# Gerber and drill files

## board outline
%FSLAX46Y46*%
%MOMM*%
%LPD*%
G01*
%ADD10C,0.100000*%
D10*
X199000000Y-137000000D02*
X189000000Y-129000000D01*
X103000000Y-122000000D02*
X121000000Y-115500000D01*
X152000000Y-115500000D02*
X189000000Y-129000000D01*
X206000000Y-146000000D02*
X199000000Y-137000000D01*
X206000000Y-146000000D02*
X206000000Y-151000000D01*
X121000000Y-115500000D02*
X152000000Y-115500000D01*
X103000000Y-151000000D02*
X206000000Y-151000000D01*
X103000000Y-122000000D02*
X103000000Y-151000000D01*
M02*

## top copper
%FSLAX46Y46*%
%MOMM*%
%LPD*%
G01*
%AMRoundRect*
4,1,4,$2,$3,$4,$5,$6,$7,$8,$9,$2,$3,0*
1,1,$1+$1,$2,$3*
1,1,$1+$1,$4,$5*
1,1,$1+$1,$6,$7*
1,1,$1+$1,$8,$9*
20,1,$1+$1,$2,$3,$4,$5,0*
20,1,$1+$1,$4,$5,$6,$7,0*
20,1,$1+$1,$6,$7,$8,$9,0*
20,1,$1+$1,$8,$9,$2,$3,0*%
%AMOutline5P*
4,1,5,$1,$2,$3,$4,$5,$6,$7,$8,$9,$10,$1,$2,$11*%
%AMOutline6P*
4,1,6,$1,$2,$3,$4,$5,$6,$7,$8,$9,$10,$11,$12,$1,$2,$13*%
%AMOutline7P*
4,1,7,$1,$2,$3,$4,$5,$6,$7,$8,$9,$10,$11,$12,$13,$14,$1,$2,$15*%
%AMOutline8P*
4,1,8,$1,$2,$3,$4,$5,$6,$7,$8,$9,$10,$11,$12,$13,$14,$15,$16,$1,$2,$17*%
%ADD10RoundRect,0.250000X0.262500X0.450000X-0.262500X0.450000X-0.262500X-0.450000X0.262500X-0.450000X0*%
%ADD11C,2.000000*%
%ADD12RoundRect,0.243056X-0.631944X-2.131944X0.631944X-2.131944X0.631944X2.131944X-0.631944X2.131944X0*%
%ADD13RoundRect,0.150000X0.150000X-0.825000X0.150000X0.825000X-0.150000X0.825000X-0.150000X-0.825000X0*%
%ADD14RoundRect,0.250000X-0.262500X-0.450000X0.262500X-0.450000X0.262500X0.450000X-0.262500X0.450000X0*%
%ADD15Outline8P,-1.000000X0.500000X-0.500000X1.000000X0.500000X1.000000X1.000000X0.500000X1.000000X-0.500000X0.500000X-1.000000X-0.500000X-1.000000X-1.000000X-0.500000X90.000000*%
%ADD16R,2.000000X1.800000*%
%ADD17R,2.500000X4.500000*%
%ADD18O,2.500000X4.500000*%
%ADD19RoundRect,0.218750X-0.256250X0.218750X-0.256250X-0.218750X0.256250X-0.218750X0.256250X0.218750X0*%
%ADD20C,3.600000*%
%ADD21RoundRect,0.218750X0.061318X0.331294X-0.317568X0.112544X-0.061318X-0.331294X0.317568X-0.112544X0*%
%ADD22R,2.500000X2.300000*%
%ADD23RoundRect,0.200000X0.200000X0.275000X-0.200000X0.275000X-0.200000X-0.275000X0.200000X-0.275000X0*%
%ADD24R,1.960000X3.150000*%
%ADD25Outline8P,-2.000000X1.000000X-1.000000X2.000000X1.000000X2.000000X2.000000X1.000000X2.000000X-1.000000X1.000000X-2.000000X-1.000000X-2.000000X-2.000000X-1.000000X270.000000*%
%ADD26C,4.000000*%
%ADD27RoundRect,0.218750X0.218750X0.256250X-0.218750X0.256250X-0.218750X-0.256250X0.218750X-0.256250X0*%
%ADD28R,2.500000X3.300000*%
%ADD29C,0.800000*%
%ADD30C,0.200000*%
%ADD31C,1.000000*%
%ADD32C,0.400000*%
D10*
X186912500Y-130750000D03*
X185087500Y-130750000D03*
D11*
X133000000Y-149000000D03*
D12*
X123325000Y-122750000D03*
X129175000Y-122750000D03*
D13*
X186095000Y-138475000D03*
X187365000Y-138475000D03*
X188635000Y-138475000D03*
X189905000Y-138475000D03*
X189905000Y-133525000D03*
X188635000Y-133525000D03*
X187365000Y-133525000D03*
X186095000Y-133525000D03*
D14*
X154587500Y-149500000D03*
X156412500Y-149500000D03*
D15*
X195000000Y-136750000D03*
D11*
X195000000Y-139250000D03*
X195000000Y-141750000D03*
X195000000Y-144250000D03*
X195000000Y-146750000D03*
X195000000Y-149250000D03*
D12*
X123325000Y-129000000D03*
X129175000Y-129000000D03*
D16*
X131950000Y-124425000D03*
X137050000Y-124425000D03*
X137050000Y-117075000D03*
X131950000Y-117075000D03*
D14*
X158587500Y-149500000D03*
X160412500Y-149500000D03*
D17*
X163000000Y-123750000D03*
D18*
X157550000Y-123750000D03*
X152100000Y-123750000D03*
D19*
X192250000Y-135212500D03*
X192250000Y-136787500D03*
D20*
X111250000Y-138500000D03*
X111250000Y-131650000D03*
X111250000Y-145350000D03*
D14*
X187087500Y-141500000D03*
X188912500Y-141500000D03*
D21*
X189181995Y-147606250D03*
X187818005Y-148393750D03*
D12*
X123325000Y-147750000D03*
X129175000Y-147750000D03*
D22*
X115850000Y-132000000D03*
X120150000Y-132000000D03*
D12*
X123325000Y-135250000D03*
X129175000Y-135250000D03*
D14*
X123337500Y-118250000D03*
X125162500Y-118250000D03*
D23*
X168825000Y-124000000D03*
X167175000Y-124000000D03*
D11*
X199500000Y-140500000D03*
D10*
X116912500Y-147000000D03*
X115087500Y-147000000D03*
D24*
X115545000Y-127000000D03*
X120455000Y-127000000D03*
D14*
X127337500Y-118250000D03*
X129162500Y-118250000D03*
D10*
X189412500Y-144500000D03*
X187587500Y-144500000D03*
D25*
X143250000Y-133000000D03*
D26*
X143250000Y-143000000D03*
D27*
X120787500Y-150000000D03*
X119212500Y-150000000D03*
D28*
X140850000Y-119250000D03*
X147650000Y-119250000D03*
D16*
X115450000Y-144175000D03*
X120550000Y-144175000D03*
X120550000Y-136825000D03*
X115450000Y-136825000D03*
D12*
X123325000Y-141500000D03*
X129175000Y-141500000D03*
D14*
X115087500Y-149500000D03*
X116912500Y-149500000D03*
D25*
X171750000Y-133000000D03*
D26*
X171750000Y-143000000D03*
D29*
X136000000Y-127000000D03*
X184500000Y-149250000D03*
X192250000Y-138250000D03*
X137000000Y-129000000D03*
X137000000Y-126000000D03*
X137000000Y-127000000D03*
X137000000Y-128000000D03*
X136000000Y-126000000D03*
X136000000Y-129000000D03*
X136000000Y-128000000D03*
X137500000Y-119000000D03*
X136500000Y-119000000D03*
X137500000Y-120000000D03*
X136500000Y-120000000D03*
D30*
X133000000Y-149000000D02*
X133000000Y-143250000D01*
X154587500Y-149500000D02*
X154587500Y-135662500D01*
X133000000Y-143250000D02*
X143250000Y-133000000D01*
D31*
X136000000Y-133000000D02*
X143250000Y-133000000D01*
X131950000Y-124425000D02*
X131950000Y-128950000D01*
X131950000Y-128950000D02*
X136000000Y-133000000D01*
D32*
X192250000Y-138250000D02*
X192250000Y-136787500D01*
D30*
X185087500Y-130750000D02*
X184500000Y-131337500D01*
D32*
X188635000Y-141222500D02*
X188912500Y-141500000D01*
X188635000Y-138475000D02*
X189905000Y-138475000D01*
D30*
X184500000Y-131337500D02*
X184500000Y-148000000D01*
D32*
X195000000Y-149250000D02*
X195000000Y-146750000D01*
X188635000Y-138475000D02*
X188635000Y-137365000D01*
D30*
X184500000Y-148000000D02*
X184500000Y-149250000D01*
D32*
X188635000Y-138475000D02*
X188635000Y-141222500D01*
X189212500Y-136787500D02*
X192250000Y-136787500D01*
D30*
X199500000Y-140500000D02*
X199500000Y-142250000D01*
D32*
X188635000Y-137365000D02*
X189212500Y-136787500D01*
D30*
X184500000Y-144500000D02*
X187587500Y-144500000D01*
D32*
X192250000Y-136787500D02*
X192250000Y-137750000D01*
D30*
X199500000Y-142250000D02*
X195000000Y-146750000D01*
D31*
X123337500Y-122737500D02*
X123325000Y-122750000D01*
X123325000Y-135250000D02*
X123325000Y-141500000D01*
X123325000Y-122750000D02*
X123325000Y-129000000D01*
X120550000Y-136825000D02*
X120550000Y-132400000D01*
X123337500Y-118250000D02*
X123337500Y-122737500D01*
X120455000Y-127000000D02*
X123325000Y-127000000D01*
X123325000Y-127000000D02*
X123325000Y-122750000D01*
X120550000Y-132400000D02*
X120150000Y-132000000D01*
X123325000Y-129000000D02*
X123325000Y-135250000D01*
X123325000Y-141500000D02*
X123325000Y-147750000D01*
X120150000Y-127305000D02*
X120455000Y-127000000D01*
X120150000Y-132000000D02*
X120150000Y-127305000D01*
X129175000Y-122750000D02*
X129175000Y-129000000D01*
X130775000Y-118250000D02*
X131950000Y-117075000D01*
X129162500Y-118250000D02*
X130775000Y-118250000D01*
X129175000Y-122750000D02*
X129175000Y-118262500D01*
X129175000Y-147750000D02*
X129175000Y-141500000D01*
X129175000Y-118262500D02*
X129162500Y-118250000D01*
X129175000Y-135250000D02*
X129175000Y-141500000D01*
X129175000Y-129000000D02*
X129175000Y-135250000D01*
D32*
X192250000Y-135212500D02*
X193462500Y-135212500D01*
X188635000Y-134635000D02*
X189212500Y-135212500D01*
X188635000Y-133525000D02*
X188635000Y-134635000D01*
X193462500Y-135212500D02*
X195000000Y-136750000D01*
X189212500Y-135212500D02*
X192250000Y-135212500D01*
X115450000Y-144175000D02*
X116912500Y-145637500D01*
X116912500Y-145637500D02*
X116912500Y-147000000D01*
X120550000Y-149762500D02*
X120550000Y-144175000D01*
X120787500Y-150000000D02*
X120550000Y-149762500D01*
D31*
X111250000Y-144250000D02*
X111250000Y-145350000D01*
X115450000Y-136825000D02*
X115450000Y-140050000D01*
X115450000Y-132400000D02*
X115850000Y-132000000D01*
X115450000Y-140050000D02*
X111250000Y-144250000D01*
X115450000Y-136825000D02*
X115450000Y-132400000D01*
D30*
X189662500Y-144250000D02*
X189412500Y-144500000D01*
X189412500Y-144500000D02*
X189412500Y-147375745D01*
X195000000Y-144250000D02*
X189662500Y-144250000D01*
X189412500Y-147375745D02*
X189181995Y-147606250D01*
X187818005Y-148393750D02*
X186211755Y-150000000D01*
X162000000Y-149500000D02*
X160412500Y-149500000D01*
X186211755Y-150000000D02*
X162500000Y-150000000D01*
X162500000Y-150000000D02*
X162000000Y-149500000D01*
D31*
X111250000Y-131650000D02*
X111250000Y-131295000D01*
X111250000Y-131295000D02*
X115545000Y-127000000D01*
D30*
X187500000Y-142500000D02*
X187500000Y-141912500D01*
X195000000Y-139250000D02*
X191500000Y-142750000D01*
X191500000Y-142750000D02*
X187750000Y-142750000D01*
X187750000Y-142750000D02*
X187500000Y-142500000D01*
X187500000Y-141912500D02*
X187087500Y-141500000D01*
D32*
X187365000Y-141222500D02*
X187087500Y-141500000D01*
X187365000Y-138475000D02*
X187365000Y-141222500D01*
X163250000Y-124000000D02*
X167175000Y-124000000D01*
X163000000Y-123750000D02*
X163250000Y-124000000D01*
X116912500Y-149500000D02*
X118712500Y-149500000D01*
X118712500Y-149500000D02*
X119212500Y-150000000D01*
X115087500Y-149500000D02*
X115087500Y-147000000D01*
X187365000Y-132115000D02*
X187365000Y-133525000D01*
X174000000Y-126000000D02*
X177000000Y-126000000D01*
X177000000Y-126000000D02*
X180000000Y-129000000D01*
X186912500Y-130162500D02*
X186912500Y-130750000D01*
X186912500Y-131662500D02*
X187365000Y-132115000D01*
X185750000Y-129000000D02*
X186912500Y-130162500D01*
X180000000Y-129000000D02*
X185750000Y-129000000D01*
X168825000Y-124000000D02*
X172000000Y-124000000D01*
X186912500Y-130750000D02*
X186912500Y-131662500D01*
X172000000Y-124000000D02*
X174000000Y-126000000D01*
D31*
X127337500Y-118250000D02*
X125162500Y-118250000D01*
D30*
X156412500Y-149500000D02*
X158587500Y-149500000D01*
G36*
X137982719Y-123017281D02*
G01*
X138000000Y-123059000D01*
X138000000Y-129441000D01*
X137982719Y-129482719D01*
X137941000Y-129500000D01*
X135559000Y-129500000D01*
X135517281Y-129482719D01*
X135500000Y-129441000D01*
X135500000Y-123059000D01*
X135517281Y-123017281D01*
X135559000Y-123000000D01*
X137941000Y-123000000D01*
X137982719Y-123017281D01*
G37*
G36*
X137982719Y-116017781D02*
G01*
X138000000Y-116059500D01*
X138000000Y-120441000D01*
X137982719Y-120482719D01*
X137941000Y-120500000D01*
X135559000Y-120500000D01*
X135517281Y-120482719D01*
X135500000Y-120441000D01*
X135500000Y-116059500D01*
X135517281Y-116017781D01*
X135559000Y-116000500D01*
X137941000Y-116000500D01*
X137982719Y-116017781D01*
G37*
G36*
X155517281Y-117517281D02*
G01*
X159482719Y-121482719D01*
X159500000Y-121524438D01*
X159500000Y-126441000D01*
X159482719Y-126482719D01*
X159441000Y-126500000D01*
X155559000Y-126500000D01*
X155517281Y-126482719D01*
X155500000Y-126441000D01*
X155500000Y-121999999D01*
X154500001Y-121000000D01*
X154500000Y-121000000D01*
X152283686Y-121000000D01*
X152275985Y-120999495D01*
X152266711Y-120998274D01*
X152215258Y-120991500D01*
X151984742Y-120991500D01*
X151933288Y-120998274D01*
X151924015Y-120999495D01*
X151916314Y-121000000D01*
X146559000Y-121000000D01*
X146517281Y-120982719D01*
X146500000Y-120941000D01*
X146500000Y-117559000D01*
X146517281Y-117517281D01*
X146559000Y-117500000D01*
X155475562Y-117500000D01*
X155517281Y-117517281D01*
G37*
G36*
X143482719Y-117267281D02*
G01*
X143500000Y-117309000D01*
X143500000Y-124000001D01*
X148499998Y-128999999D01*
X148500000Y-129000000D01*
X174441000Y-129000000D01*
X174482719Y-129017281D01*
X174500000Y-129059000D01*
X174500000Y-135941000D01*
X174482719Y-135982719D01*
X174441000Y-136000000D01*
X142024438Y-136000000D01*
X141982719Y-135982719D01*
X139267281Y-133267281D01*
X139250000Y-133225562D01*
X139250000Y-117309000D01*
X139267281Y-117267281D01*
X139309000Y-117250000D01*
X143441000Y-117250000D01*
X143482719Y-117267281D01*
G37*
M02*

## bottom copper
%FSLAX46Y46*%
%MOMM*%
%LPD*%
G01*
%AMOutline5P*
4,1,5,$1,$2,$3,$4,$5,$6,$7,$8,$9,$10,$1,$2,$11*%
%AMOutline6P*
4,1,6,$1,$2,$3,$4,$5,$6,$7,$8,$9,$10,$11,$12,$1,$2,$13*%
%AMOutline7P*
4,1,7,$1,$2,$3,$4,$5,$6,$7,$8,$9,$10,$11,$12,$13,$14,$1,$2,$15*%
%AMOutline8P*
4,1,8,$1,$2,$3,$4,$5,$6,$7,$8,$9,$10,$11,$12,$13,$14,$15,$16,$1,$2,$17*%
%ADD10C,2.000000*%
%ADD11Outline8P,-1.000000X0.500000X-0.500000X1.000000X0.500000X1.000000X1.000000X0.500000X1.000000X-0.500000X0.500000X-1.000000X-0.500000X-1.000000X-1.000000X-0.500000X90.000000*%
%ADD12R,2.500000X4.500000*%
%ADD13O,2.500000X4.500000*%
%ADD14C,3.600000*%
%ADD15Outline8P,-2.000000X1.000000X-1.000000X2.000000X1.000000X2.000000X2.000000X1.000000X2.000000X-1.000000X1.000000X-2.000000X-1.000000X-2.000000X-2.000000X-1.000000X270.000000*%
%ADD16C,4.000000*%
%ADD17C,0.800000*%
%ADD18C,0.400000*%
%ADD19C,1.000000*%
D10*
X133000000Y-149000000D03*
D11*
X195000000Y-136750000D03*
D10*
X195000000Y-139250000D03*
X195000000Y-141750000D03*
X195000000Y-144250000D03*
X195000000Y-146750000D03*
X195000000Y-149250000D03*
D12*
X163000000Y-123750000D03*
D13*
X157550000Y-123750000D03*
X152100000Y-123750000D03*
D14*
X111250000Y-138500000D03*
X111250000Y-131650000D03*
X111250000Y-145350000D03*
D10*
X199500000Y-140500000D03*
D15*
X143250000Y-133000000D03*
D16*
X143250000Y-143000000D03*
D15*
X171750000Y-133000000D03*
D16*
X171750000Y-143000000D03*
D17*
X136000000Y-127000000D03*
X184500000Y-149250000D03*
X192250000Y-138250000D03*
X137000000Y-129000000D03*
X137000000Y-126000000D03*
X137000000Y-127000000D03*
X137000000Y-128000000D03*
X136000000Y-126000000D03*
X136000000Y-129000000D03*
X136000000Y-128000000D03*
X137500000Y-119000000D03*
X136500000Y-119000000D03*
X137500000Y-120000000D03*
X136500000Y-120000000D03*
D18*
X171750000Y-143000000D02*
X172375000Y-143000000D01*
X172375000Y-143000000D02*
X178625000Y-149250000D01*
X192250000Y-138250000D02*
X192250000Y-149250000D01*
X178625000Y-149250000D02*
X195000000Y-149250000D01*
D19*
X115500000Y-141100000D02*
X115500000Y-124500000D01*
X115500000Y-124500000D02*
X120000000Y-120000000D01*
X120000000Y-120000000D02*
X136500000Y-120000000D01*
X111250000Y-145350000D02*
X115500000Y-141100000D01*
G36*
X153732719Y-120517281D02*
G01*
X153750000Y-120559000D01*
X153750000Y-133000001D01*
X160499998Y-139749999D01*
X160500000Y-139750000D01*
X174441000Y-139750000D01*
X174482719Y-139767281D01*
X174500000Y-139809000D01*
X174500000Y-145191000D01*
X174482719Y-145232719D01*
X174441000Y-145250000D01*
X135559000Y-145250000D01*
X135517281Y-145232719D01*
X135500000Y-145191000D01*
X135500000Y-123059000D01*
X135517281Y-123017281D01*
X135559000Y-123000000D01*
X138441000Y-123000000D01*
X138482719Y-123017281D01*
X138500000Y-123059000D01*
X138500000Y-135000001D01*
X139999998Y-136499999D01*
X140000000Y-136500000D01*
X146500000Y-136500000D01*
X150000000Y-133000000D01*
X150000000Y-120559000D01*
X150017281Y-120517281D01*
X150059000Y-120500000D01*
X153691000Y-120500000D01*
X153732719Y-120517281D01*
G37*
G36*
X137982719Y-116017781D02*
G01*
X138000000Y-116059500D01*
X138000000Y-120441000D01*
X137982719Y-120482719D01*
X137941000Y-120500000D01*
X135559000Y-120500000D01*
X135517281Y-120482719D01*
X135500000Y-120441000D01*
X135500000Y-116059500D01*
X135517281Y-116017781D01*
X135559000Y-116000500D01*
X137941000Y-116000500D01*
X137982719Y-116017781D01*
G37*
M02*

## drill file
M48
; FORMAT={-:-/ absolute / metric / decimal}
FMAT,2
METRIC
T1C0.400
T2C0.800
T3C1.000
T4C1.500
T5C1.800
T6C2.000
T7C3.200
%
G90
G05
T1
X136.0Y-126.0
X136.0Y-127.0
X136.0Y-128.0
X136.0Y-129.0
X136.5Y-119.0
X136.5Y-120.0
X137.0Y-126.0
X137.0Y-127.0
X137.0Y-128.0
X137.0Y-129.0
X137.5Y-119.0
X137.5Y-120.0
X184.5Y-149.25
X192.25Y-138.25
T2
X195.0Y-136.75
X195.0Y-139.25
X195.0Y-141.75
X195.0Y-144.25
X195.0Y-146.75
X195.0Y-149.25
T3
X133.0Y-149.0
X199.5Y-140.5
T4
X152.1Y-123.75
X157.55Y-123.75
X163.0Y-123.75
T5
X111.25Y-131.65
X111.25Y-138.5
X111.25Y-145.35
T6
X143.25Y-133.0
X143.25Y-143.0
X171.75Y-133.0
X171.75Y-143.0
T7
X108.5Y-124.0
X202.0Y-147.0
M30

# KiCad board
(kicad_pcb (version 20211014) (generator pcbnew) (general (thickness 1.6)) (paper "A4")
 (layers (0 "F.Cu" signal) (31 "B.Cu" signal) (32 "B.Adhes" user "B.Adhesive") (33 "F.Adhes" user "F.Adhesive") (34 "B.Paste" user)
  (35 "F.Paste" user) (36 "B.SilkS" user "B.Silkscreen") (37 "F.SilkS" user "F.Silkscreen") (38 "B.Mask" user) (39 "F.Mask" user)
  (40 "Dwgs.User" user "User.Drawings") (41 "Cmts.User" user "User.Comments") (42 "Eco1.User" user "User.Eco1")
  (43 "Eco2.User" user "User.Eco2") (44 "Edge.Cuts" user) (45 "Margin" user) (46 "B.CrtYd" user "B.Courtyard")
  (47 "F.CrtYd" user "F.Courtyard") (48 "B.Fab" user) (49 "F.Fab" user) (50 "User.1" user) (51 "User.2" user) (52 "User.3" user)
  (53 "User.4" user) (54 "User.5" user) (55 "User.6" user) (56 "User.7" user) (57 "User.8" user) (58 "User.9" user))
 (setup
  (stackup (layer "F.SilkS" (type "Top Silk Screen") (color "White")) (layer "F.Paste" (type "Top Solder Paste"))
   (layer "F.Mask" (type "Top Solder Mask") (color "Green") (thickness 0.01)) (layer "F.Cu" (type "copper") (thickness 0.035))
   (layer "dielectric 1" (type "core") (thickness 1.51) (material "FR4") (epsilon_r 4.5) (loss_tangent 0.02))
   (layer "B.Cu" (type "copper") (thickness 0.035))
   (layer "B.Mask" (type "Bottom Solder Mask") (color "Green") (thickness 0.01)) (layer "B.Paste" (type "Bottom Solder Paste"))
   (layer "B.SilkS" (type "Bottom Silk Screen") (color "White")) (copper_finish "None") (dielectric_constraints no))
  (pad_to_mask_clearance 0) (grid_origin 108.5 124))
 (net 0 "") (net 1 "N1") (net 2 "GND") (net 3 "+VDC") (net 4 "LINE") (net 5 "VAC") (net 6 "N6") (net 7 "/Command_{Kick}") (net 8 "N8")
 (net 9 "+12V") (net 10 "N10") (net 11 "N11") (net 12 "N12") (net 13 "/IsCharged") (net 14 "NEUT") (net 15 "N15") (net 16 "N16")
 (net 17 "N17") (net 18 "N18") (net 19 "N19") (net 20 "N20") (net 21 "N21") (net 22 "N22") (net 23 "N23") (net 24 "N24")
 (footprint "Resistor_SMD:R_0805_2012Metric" (layer "F.Cu") (at 186 130.75 180)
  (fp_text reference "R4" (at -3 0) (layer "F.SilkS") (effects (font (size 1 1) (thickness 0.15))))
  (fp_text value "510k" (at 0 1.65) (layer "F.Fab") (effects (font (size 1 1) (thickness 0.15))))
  (pad "1" smd roundrect (at -0.9125 0 180) (size 1.025 1.4) (layers "F.Cu" "F.Paste" "F.Mask") (roundrect_rratio 0.243902439) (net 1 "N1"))
  (pad "2" smd roundrect (at 0.9125 0 180) (size 1.025 1.4) (layers "F.Cu" "F.Paste" "F.Mask") (roundrect_rratio 0.243902439) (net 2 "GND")))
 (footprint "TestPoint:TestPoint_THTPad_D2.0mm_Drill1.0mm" (layer "F.Cu") (at 133 149)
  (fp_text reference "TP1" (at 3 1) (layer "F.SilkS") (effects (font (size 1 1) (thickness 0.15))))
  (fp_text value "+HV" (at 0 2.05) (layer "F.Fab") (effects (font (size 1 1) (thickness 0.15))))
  (pad "1" thru_hole circle (at 0 0) (size 2 2) (drill 1) (layers *.Cu *.Mask) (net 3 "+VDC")))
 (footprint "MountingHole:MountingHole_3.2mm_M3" (layer "F.Cu") (at 202 147)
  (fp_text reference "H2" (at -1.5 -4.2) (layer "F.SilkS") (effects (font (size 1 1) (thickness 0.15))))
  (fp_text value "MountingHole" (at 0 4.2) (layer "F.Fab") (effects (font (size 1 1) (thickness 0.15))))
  (pad "" np_thru_hole circle (at 0 0) (size 3.2 3.2) (drill 3.2) (layers *.Cu *.Mask)))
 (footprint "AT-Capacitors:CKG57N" (layer "F.Cu") (at 126.25 122.75)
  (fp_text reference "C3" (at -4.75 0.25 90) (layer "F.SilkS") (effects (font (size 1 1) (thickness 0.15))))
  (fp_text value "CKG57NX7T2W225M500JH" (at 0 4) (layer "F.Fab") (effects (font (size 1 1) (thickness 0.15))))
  (pad "1" smd roundrect (at -2.925 0) (size 1.75 4.75) (layers "F.Cu" "F.Paste" "F.Mask") (roundrect_rratio 0.1388891429) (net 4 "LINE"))
  (pad "2" smd roundrect (at 2.925 0) (size 1.75 4.75) (layers "F.Cu" "F.Paste" "F.Mask") (roundrect_rratio 0.1388891429) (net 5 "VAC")))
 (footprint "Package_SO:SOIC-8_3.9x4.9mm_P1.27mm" (layer "F.Cu") (at 188 136 90)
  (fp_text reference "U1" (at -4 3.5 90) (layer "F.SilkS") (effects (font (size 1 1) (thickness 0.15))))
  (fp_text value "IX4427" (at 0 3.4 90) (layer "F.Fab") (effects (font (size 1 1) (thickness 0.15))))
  (pad "1" smd roundrect (at -2.475 -1.905 90) (size 1.95 0.6) (layers "F.Cu" "F.Paste" "F.Mask") (roundrect_rratio 0.25) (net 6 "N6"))
  (pad "2" smd roundrect (at -2.475 -0.635 90) (size 1.95 0.6) (layers "F.Cu" "F.Paste" "F.Mask") (roundrect_rratio 0.25)
   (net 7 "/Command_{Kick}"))
  (pad "3" smd roundrect (at -2.475 0.635 90) (size 1.95 0.6) (layers "F.Cu" "F.Paste" "F.Mask") (roundrect_rratio 0.25) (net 2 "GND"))
  (pad "4" smd roundrect (at -2.475 1.905 90) (size 1.95 0.6) (layers "F.Cu" "F.Paste" "F.Mask") (roundrect_rratio 0.25) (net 2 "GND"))
  (pad "5" smd roundrect (at 2.475 1.905 90) (size 1.95 0.6) (layers "F.Cu" "F.Paste" "F.Mask") (roundrect_rratio 0.25) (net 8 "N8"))
  (pad "6" smd roundrect (at 2.475 0.635 90) (size 1.95 0.6) (layers "F.Cu" "F.Paste" "F.Mask") (roundrect_rratio 0.25) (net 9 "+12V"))
  (pad "7" smd roundrect (at 2.475 -0.635 90) (size 1.95 0.6) (layers "F.Cu" "F.Paste" "F.Mask") (roundrect_rratio 0.25) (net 1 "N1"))
  (pad "8" smd roundrect (at 2.475 -1.905 90) (size 1.95 0.6) (layers "F.Cu" "F.Paste" "F.Mask") (roundrect_rratio 0.25) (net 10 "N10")))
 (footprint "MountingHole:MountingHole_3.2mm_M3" (layer "F.Cu") (at 108.5 124)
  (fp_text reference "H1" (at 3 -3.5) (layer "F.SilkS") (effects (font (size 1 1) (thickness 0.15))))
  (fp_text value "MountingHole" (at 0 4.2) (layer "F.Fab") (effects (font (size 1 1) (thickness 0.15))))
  (pad "" np_thru_hole circle (at 0 0) (size 3.2 3.2) (drill 3.2) (layers *.Cu *.Mask)))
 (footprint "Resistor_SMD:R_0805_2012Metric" (layer "F.Cu") (at 155.5 149.5)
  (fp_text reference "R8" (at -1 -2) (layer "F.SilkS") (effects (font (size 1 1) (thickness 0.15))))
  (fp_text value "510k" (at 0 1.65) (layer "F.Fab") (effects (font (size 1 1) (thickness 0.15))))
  (pad "1" smd roundrect (at -0.9125 0) (size 1.025 1.4) (layers "F.Cu" "F.Paste" "F.Mask") (roundrect_rratio 0.243902439) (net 3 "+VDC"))
  (pad "2" smd roundrect (at 0.9125 0) (size 1.025 1.4) (layers "F.Cu" "F.Paste" "F.Mask") (roundrect_rratio 0.243902439) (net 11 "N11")))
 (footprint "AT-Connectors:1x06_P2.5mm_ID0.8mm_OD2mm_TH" (layer "F.Cu") (at 195 143 -90)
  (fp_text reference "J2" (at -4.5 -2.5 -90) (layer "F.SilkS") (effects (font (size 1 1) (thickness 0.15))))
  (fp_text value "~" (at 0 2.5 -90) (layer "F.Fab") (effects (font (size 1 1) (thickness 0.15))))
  (pad "1" thru_hole roundrect (at -6.25 0 90) (size 2 2) (drill 0.8) (layers *.Cu *.Mask) (roundrect_rratio 0) (chamfer_ratio 0.25)
   (chamfer top_left top_right bottom_left bottom_right) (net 9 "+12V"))
  (pad "2" thru_hole circle (at -3.75 0 90) (size 2 2) (drill 0.8) (layers *.Cu *.Mask) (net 7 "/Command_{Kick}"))
  (pad "3" thru_hole circle (at -1.25 0 90) (size 2 2) (drill 0.8) (layers *.Cu *.Mask) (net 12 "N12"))
  (pad "4" thru_hole circle (at 1.25 0 90) (size 2 2) (drill 0.8) (layers *.Cu *.Mask) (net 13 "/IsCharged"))
  (pad "5" thru_hole circle (at 3.75 0 90) (size 2 2) (drill 0.8) (layers *.Cu *.Mask) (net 2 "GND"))
  (pad "6" thru_hole circle (at 6.25 0 90) (size 2 2) (drill 0.8) (layers *.Cu *.Mask) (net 2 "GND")))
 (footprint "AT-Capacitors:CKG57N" (layer "F.Cu") (at 126.25 129)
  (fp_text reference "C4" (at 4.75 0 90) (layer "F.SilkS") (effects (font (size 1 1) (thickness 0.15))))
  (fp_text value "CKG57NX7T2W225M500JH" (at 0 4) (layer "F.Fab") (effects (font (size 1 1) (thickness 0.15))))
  (pad "1" smd roundrect (at -2.925 0) (size 1.75 4.75) (layers "F.Cu" "F.Paste" "F.Mask") (roundrect_rratio 0.1388891429) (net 4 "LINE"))
  (pad "2" smd roundrect (at 2.925 0) (size 1.75 4.75) (layers "F.Cu" "F.Paste" "F.Mask") (roundrect_rratio 0.1388891429) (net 5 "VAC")))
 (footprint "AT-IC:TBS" (layer "F.Cu") (at 134.5 120.75 180)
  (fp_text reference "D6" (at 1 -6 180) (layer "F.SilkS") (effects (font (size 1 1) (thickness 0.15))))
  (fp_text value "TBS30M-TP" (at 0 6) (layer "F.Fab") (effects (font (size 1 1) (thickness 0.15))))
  (pad "1" smd rect (at 2.55 -3.675 180) (size 2 1.8) (layers "F.Cu" "F.Paste" "F.Mask") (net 3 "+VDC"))
  (pad "2" smd rect (at -2.55 -3.675 180) (size 2 1.8) (layers "F.Cu" "F.Paste" "F.Mask") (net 2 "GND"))
  (pad "3" smd rect (at -2.55 3.675) (size 2 1.8) (layers "F.Cu" "F.Paste" "F.Mask") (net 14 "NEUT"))
  (pad "4" smd rect (at 2.55 3.675) (size 2 1.8) (layers "F.Cu" "F.Paste" "F.Mask") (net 5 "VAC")))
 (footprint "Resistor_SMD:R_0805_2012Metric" (layer "F.Cu") (at 159.5 149.5)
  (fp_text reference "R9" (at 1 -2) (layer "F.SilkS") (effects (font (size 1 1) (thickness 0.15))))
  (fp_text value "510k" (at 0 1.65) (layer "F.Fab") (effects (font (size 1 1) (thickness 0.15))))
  (pad "1" smd roundrect (at -0.9125 0) (size 1.025 1.4) (layers "F.Cu" "F.Paste" "F.Mask") (roundrect_rratio 0.243902439) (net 11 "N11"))
  (pad "2" smd roundrect (at 0.9125 0) (size 1.025 1.4) (layers "F.Cu" "F.Paste" "F.Mask") (roundrect_rratio 0.243902439) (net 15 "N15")))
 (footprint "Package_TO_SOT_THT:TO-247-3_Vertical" (layer "F.Cu") (at 163 123.75 180)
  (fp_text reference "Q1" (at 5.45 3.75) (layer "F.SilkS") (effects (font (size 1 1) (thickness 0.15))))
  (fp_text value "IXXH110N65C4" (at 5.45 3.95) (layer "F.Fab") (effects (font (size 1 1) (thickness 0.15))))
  (pad "1" thru_hole rect (at 0 0 180) (size 2.5 4.5) (drill 1.5) (layers *.Cu *.Mask) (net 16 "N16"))
  (pad "2" thru_hole oval (at 5.45 0 180) (size 2.5 4.5) (drill 1.5) (layers *.Cu *.Mask) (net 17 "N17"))
  (pad "3" thru_hole oval (at 10.9 0 180) (size 2.5 4.5) (drill 1.5) (layers *.Cu *.Mask) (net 2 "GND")))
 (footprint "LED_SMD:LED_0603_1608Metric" (layer "F.Cu") (at 192.25 136 -90)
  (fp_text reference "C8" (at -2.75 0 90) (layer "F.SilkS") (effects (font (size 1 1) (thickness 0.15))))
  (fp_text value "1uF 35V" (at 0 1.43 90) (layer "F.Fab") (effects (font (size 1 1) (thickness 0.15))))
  (pad "1" smd roundrect (at -0.7875 0 270) (size 0.875 0.95) (layers "F.Cu" "F.Paste" "F.Mask") (roundrect_rratio 0.25) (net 9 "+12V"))
  (pad "2" smd roundrect (at 0.7875 0 270) (size 0.875 0.95) (layers "F.Cu" "F.Paste" "F.Mask") (roundrect_rratio 0.25) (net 2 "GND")))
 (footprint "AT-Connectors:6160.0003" (layer "F.Cu") (at 111.25 138.5 -90)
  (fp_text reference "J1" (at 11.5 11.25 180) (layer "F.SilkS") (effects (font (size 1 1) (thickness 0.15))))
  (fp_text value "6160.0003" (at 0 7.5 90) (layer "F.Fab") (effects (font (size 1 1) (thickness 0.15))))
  (pad "G" thru_hole circle (at 0 0 270) (size 3.6 3.6) (drill 1.8) (layers *.Cu *.Mask) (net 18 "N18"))
  (pad "L" thru_hole circle (at -6.85 0 270) (size 3.6 3.6) (drill 1.8) (layers *.Cu *.Mask) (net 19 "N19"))
  (pad "N" thru_hole circle (at 6.85 0 270) (size 3.6 3.6) (drill 1.8) (layers *.Cu *.Mask) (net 14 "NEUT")))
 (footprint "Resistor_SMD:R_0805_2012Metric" (layer "F.Cu") (at 188 141.5)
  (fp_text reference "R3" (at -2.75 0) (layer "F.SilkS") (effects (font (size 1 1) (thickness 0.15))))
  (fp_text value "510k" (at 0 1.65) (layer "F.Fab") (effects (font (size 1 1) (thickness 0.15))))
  (pad "1" smd roundrect (at -0.9125 0) (size 1.025 1.4) (layers "F.Cu" "F.Paste" "F.Mask") (roundrect_rratio 0.243902439)
   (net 7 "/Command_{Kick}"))
  (pad "2" smd roundrect (at 0.9125 0) (size 1.025 1.4) (layers "F.Cu" "F.Paste" "F.Mask") (roundrect_rratio 0.243902439) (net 2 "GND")))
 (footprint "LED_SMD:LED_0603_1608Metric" (layer "F.Cu") (at 188.5 148 -150)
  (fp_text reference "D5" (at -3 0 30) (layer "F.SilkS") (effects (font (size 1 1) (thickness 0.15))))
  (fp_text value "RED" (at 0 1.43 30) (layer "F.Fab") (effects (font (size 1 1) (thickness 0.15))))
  (pad "1" smd roundrect (at -0.7875 0 210) (size 0.875 0.95) (layers "F.Cu" "F.Paste" "F.Mask") (roundrect_rratio 0.25)
   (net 13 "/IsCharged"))
  (pad "2" smd roundrect (at 0.7875 0 210) (size 0.875 0.95) (layers "F.Cu" "F.Paste" "F.Mask") (roundrect_rratio 0.25) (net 15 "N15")))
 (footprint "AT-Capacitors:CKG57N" (layer "F.Cu") (at 126.25 147.75)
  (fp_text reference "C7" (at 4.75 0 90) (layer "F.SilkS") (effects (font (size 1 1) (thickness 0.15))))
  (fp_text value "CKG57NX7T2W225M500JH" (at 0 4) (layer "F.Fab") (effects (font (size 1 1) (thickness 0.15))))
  (pad "1" smd roundrect (at -2.925 0) (size 1.75 4.75) (layers "F.Cu" "F.Paste" "F.Mask") (roundrect_rratio 0.1388891429) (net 4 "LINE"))
  (pad "2" smd roundrect (at 2.925 0) (size 1.75 4.75) (layers "F.Cu" "F.Paste" "F.Mask") (roundrect_rratio 0.1388891429) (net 5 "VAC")))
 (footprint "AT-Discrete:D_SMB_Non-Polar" (layer "F.Cu") (at 118 132)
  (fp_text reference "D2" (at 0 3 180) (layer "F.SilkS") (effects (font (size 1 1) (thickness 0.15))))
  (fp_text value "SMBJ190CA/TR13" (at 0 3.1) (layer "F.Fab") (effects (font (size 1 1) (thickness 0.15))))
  (pad "1" smd rect (at -2.15 0) (size 2.5 2.3) (layers "F.Cu" "F.Paste" "F.Mask") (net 14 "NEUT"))
  (pad "2" smd rect (at 2.15 0) (size 2.5 2.3) (layers "F.Cu" "F.Paste" "F.Mask") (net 4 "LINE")))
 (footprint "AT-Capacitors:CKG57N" (layer "F.Cu") (at 126.25 135.25)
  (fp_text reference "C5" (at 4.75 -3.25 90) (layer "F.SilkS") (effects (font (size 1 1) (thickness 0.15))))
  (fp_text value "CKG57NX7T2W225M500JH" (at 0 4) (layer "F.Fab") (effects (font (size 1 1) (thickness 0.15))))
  (pad "1" smd roundrect (at -2.925 0) (size 1.75 4.75) (layers "F.Cu" "F.Paste" "F.Mask") (roundrect_rratio 0.1388891429) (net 4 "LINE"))
  (pad "2" smd roundrect (at 2.925 0) (size 1.75 4.75) (layers "F.Cu" "F.Paste" "F.Mask") (roundrect_rratio 0.1388891429) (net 5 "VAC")))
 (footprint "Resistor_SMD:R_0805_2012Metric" (layer "F.Cu") (at 124.25 118.25)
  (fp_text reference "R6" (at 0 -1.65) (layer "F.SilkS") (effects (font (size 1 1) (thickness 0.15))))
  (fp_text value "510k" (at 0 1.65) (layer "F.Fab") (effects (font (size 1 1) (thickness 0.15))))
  (pad "1" smd roundrect (at -0.9125 0) (size 1.025 1.4) (layers "F.Cu" "F.Paste" "F.Mask") (roundrect_rratio 0.243902439) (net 4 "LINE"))
  (pad "2" smd roundrect (at 0.9125 0) (size 1.025 1.4) (layers "F.Cu" "F.Paste" "F.Mask") (roundrect_rratio 0.243902439) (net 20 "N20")))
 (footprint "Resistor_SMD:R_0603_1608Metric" (layer "F.Cu") (at 168 124 180)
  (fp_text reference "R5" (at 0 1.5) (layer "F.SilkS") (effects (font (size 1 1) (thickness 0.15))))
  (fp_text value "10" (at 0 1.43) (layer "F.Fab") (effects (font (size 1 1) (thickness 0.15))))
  (pad "1" smd roundrect (at -0.825 0 180) (size 0.8 0.95) (layers "F.Cu" "F.Paste" "F.Mask") (roundrect_rratio 0.25) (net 1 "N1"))
  (pad "2" smd roundrect (at 0.825 0 180) (size 0.8 0.95) (layers "F.Cu" "F.Paste" "F.Mask") (roundrect_rratio 0.25) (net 16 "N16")))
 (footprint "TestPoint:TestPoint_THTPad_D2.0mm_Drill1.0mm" (layer "F.Cu") (at 199.5 140.5)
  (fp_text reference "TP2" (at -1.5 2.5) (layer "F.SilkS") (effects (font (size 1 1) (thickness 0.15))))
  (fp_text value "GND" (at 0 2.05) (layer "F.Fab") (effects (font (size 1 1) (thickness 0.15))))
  (pad "1" thru_hole circle (at 0 0) (size 2 2) (drill 1) (layers *.Cu *.Mask) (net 2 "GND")))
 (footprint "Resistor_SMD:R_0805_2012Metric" (layer "F.Cu") (at 116 147 180)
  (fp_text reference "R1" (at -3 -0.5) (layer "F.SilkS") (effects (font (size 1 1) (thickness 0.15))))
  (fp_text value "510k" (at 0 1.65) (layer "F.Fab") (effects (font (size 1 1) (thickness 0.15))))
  (pad "1" smd roundrect (at -0.9125 0 180) (size 1.025 1.4) (layers "F.Cu" "F.Paste" "F.Mask") (roundrect_rratio 0.243902439)
   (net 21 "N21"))
  (pad "2" smd roundrect (at 0.9125 0 180) (size 1.025 1.4) (layers "F.Cu" "F.Paste" "F.Mask") (roundrect_rratio 0.243902439) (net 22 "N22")))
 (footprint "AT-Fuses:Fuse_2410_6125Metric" (layer "F.Cu") (at 118 127)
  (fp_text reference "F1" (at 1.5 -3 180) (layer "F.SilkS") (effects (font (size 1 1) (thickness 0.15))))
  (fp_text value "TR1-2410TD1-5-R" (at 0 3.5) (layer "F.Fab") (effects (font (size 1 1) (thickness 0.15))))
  (pad "1" smd rect (at -2.455 0) (size 1.96 3.15) (layers "F.Cu" "F.Paste" "F.Mask") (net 19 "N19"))
  (pad "2" smd rect (at 2.455 0) (size 1.96 3.15) (layers "F.Cu" "F.Paste" "F.Mask") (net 4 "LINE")))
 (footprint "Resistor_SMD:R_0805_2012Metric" (layer "F.Cu") (at 128.25 118.25)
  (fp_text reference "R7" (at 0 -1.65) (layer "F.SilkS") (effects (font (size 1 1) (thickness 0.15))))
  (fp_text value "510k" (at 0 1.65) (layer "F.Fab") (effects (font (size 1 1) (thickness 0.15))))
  (pad "1" smd roundrect (at -0.9125 0) (size 1.025 1.4) (layers "F.Cu" "F.Paste" "F.Mask") (roundrect_rratio 0.243902439) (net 20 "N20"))
  (pad "2" smd roundrect (at 0.9125 0) (size 1.025 1.4) (layers "F.Cu" "F.Paste" "F.Mask") (roundrect_rratio 0.243902439) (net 5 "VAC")))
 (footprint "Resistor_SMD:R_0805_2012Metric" (layer "F.Cu") (at 188.5 144.5 180)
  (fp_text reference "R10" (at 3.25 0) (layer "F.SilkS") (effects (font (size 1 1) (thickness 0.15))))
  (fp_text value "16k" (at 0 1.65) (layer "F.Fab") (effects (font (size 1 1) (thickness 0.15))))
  (pad "1" smd roundrect (at -0.9125 0 180) (size 1.025 1.4) (layers "F.Cu" "F.Paste" "F.Mask") (roundrect_rratio 0.243902439)
   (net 13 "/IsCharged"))
  (pad "2" smd roundrect (at 0.9125 0 180) (size 1.025 1.4) (layers "F.Cu" "F.Paste" "F.Mask") (roundrect_rratio 0.243902439) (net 2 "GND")))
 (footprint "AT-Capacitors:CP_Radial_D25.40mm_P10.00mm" (layer "F.Cu") (at 143.25 138 -90)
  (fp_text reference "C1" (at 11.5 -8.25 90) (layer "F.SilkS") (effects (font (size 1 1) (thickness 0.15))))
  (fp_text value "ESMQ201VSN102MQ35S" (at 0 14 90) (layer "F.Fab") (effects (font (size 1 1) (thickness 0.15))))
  (pad "1" thru_hole roundrect (at -5 0 270) (size 4 4) (drill 2) (layers *.Cu *.Mask) (roundrect_rratio 0) (chamfer_ratio 0.25)
   (chamfer top_left top_right bottom_left bottom_right) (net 3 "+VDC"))
  (pad "2" thru_hole circle (at 5 0 270) (size 4 4) (drill 2) (layers *.Cu *.Mask) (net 2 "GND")))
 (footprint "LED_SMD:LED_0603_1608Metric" (layer "F.Cu") (at 120 150 180)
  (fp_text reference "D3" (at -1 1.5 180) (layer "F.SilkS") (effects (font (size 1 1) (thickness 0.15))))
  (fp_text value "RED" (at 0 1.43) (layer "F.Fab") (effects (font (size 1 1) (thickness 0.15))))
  (pad "1" smd roundrect (at -0.7875 0 180) (size 0.875 0.95) (layers "F.Cu" "F.Paste" "F.Mask") (roundrect_rratio 0.25) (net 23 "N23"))
  (pad "2" smd roundrect (at 0.7875 0 180) (size 0.875 0.95) (layers "F.Cu" "F.Paste" "F.Mask") (roundrect_rratio 0.25) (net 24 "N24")))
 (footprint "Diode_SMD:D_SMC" (layer "F.Cu") (at 144.25 119.25)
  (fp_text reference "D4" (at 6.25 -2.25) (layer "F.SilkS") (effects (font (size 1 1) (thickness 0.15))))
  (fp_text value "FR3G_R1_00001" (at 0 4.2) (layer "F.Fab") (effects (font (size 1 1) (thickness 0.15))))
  (pad "1" smd rect (at -3.4 0 90) (size 3.3 2.5) (layers "F.Cu" "F.Paste" "F.Mask") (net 3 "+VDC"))
  (pad "2" smd rect (at 3.4 0 90) (size 3.3 2.5) (layers "F.Cu" "F.Paste" "F.Mask") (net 17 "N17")))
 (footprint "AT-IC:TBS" (layer "F.Cu") (at 118 140.5 180)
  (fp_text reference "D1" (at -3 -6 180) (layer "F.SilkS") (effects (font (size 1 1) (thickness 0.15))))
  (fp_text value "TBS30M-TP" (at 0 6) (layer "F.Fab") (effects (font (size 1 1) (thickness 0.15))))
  (pad "1" smd rect (at 2.55 -3.675 180) (size 2 1.8) (layers "F.Cu" "F.Paste" "F.Mask") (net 21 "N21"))
  (pad "2" smd rect (at -2.55 -3.675 180) (size 2 1.8) (layers "F.Cu" "F.Paste" "F.Mask") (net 23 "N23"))
  (pad "3" smd rect (at -2.55 3.675) (size 2 1.8) (layers "F.Cu" "F.Paste" "F.Mask") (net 4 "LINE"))
  (pad "4" smd rect (at 2.55 3.675) (size 2 1.8) (layers "F.Cu" "F.Paste" "F.Mask") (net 14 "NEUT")))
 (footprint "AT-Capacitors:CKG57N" (layer "F.Cu") (at 126.25 141.5)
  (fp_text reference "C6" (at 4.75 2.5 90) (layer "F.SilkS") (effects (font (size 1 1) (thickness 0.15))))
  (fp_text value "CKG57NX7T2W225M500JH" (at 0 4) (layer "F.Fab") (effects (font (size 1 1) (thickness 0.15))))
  (pad "1" smd roundrect (at -2.925 0) (size 1.75 4.75) (layers "F.Cu" "F.Paste" "F.Mask") (roundrect_rratio 0.1388891429) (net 4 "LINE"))
  (pad "2" smd roundrect (at 2.925 0) (size 1.75 4.75) (layers "F.Cu" "F.Paste" "F.Mask") (roundrect_rratio 0.1388891429) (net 5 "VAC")))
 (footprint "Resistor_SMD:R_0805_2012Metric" (layer "F.Cu") (at 116 149.5)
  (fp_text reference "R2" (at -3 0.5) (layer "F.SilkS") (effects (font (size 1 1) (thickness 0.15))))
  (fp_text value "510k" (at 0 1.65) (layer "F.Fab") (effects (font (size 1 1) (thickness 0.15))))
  (pad "1" smd roundrect (at -0.9125 0) (size 1.025 1.4) (layers "F.Cu" "F.Paste" "F.Mask") (roundrect_rratio 0.243902439) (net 22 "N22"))
  (pad "2" smd roundrect (at 0.9125 0) (size 1.025 1.4) (layers "F.Cu" "F.Paste" "F.Mask") (roundrect_rratio 0.243902439) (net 24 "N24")))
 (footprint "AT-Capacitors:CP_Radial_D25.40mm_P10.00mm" (layer "F.Cu") (at 171.75 138 -90)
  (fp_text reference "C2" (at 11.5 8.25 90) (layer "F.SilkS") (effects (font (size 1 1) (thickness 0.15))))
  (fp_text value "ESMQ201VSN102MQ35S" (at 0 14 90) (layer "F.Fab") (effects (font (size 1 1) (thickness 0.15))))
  (pad "1" thru_hole roundrect (at -5 0 270) (size 4 4) (drill 2) (layers *.Cu *.Mask) (roundrect_rratio 0) (chamfer_ratio 0.25)
   (chamfer top_left top_right bottom_left bottom_right) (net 3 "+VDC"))
  (pad "2" thru_hole circle (at 5 0 270) (size 4 4) (drill 2) (layers *.Cu *.Mask) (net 2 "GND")))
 (gr_line (start 199 137) (end 189 129) (layer "Edge.Cuts") (width 0.1))
 (gr_line (start 103 122) (end 121 115.5) (layer "Edge.Cuts") (width 0.1))
 (gr_line (start 152 115.5) (end 189 129) (layer "Edge.Cuts") (width 0.1))
 (gr_line (start 206 146) (end 199 137) (layer "Edge.Cuts") (width 0.1))
 (gr_line (start 206 146) (end 206 151) (layer "Edge.Cuts") (width 0.1))
 (gr_line (start 121 115.5) (end 152 115.5) (layer "Edge.Cuts") (width 0.1))
 (gr_line (start 103 151) (end 206 151) (layer "Edge.Cuts") (width 0.1))
 (gr_line (start 103 122) (end 103 151) (layer "Edge.Cuts") (width 0.1))
 (segment (start 133 149) (end 133 143.25) (width 0.2) (layer "F.Cu") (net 3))
 (segment (start 154.5875 149.5) (end 154.5875 135.6625) (width 0.2) (layer "F.Cu") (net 3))
 (segment (start 133 143.25) (end 143.25 133) (width 0.2) (layer "F.Cu") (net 3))
 (segment (start 136 133) (end 143.25 133) (width 1) (layer "F.Cu") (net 3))
 (segment (start 131.95 124.425) (end 131.95 128.95) (width 1) (layer "F.Cu") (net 3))
 (segment (start 131.95 128.95) (end 136 133) (width 1) (layer "F.Cu") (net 3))
 (segment (start 192.25 138.25) (end 192.25 136.7875) (width 0.4) (layer "F.Cu") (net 2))
 (segment (start 185.0875 130.75) (end 184.5 131.3375) (width 0.2) (layer "F.Cu") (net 2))
 (segment (start 188.635 141.2225) (end 188.9125 141.5) (width 0.4) (layer "F.Cu") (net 2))
 (segment (start 188.635 138.475) (end 189.905 138.475) (width 0.4) (layer "F.Cu") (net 2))
 (segment (start 184.5 131.3375) (end 184.5 148) (width 0.2) (layer "F.Cu") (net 2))
 (segment (start 195 149.25) (end 195 146.75) (width 0.4) (layer "F.Cu") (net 2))
 (segment (start 188.635 138.475) (end 188.635 137.365) (width 0.4) (layer "F.Cu") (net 2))
 (segment (start 184.5 148) (end 184.5 149.25) (width 0.2) (layer "F.Cu") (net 2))
 (segment (start 188.635 138.475) (end 188.635 141.2225) (width 0.4) (layer "F.Cu") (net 2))
 (segment (start 189.2125 136.7875) (end 192.25 136.7875) (width 0.4) (layer "F.Cu") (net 2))
 (segment (start 199.5 140.5) (end 199.5 142.25) (width 0.2) (layer "F.Cu") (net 2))
 (segment (start 188.635 137.365) (end 189.2125 136.7875) (width 0.4) (layer "F.Cu") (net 2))
 (segment (start 184.5 144.5) (end 187.5875 144.5) (width 0.2) (layer "F.Cu") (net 2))
 (segment (start 192.25 136.7875) (end 192.25 137.75) (width 0.4) (layer "F.Cu") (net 2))
 (segment (start 199.5 142.25) (end 195 146.75) (width 0.2) (layer "F.Cu") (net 2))
 (via (at 136 127) (size 0.8) (drill 0.4) (layers "F.Cu" "B.Cu") (free) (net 2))
 (via (at 184.5 149.25) (size 0.8) (drill 0.4) (layers "F.Cu" "B.Cu") (free) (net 2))
 (via (at 192.25 138.25) (size 0.8) (drill 0.4) (layers "F.Cu" "B.Cu") (free) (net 2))
 (via (at 137 129) (size 0.8) (drill 0.4) (layers "F.Cu" "B.Cu") (free) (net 2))
 (via (at 137 126) (size 0.8) (drill 0.4) (layers "F.Cu" "B.Cu") (free) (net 2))
 (via (at 137 127) (size 0.8) (drill 0.4) (layers "F.Cu" "B.Cu") (free) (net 2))
 (via (at 137 128) (size 0.8) (drill 0.4) (layers "F.Cu" "B.Cu") (free) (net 2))
 (via (at 136 126) (size 0.8) (drill 0.4) (layers "F.Cu" "B.Cu") (free) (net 2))
 (via (at 136 129) (size 0.8) (drill 0.4) (layers "F.Cu" "B.Cu") (free) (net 2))
 (via (at 136 128) (size 0.8) (drill 0.4) (layers "F.Cu" "B.Cu") (free) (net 2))
 (segment (start 171.75 143) (end 172.375 143) (width 0.4) (layer "B.Cu") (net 2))
 (segment (start 172.375 143) (end 178.625 149.25) (width 0.4) (layer "B.Cu") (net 2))
 (segment (start 192.25 138.25) (end 192.25 149.25) (width 0.4) (layer "B.Cu") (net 2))
 (segment (start 178.625 149.25) (end 195 149.25) (width 0.4) (layer "B.Cu") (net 2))
 (segment (start 123.3375 122.7375) (end 123.325 122.75) (width 1) (layer "F.Cu") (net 4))
 (segment (start 123.325 135.25) (end 123.325 141.5) (width 1) (layer "F.Cu") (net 4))
 (segment (start 123.325 122.75) (end 123.325 129) (width 1) (layer "F.Cu") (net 4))
 (segment (start 120.55 136.825) (end 120.55 132.4) (width 1) (layer "F.Cu") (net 4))
 (segment (start 123.3375 118.25) (end 123.3375 122.7375) (width 1) (layer "F.Cu") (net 4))
 (segment (start 120.455 127) (end 123.325 127) (width 1) (layer "F.Cu") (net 4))
 (segment (start 123.325 127) (end 123.325 122.75) (width 1) (layer "F.Cu") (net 4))
 (segment (start 120.55 132.4) (end 120.15 132) (width 1) (layer "F.Cu") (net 4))
 (segment (start 123.325 129) (end 123.325 135.25) (width 1) (layer "F.Cu") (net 4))
 (segment (start 123.325 141.5) (end 123.325 147.75) (width 1) (layer "F.Cu") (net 4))
 (segment (start 120.15 127.305) (end 120.455 127) (width 1) (layer "F.Cu") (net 4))
 (segment (start 120.15 132) (end 120.15 127.305) (width 1) (layer "F.Cu") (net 4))
 (segment (start 129.175 122.75) (end 129.175 129) (width 1) (layer "F.Cu") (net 5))
 (segment (start 130.775 118.25) (end 131.95 117.075) (width 1) (layer "F.Cu") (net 5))
 (segment (start 129.1625 118.25) (end 130.775 118.25) (width 1) (layer "F.Cu") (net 5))
 (segment (start 129.175 122.75) (end 129.175 118.2625) (width 1) (layer "F.Cu") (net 5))
 (segment (start 129.175 147.75) (end 129.175 141.5) (width 1) (layer "F.Cu") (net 5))
 (segment (start 129.175 118.2625) (end 129.1625 118.25) (width 1) (layer "F.Cu") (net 5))
 (segment (start 129.175 135.25) (end 129.175 141.5) (width 1) (layer "F.Cu") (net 5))
 (segment (start 129.175 129) (end 129.175 135.25) (width 1) (layer "F.Cu") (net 5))
 (segment (start 192.25 135.2125) (end 193.4625 135.2125) (width 0.4) (layer "F.Cu") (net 9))
 (segment (start 188.635 134.635) (end 189.2125 135.2125) (width 0.4) (layer "F.Cu") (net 9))
 (segment (start 188.635 133.525) (end 188.635 134.635) (width 0.4) (layer "F.Cu") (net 9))
 (segment (start 193.4625 135.2125) (end 195 136.75) (width 0.4) (layer "F.Cu") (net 9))
 (segment (start 189.2125 135.2125) (end 192.25 135.2125) (width 0.4) (layer "F.Cu") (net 9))
 (segment (start 115.45 144.175) (end 116.9125 145.6375) (width 0.4) (layer "F.Cu") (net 21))
 (segment (start 116.9125 145.6375) (end 116.9125 147) (width 0.4) (layer "F.Cu") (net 21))
 (segment (start 120.55 149.7625) (end 120.55 144.175) (width 0.4) (layer "F.Cu") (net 23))
 (segment (start 120.7875 150) (end 120.55 149.7625) (width 0.4) (layer "F.Cu") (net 23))
 (segment (start 111.25 144.25) (end 111.25 145.35) (width 1) (layer "F.Cu") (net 14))
 (segment (start 115.45 136.825) (end 115.45 140.05) (width 1) (layer "F.Cu") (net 14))
 (segment (start 115.45 132.4) (end 115.85 132) (width 1) (layer "F.Cu") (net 14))
 (segment (start 115.45 140.05) (end 111.25 144.25) (width 1) (layer "F.Cu") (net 14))
 (segment (start 115.45 136.825) (end 115.45 132.4) (width 1) (layer "F.Cu") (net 14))
 (via (at 137.5 119) (size 0.8) (drill 0.4) (layers "F.Cu" "B.Cu") (free) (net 14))
 (via (at 136.5 119) (size 0.8) (drill 0.4) (layers "F.Cu" "B.Cu") (free) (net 14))
 (via (at 137.5 120) (size 0.8) (drill 0.4) (layers "F.Cu" "B.Cu") (free) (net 14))
 (via (at 136.5 120) (size 0.8) (drill 0.4) (layers "F.Cu" "B.Cu") (free) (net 14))
 (segment (start 115.5 141.1) (end 115.5 124.5) (width 1) (layer "B.Cu") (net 14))
 (segment (start 115.5 124.5) (end 120 120) (width 1) (layer "B.Cu") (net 14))
 (segment (start 120 120) (end 136.5 120) (width 1) (layer "B.Cu") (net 14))
 (segment (start 111.25 145.35) (end 115.5 141.1) (width 1) (layer "B.Cu") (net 14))
 (segment (start 189.6625 144.25) (end 189.4125 144.5) (width 0.2) (layer "F.Cu") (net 13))
 (segment (start 189.4125 144.5) (end 189.4125 147.375745) (width 0.2) (layer "F.Cu") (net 13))
 (segment (start 195 144.25) (end 189.6625 144.25) (width 0.2) (layer "F.Cu") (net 13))
 (segment (start 189.4125 147.375745) (end 189.181995 147.60625) (width 0.2) (layer "F.Cu") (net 13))
 (segment (start 187.818005 148.39375) (end 186.211755 150) (width 0.2) (layer "F.Cu") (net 15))
 (segment (start 162 149.5) (end 160.4125 149.5) (width 0.2) (layer "F.Cu") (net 15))
 (segment (start 186.211755 150) (end 162.5 150) (width 0.2) (layer "F.Cu") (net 15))
 (segment (start 162.5 150) (end 162 149.5) (width 0.2) (layer "F.Cu") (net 15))
 (segment (start 111.25 131.65) (end 111.25 131.295) (width 1) (layer "F.Cu") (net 19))
 (segment (start 111.25 131.295) (end 115.545 127) (width 1) (layer "F.Cu") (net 19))
 (segment (start 187.5 142.5) (end 187.5 141.9125) (width 0.2) (layer "F.Cu") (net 7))
 (segment (start 195 139.25) (end 191.5 142.75) (width 0.2) (layer "F.Cu") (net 7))
 (segment (start 191.5 142.75) (end 187.75 142.75) (width 0.2) (layer "F.Cu") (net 7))
 (segment (start 187.75 142.75) (end 187.5 142.5) (width 0.2) (layer "F.Cu") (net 7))
 (segment (start 187.5 141.9125) (end 187.0875 141.5) (width 0.2) (layer "F.Cu") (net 7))
 (segment (start 187.365 141.2225) (end 187.0875 141.5) (width 0.4) (layer "F.Cu") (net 7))
 (segment (start 187.365 138.475) (end 187.365 141.2225) (width 0.4) (layer "F.Cu") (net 7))
 (segment (start 163.25 124) (end 167.175 124) (width 0.4) (layer "F.Cu") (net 16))
 (segment (start 163 123.75) (end 163.25 124) (width 0.4) (layer "F.Cu") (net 16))
 (segment (start 116.9125 149.5) (end 118.7125 149.5) (width 0.4) (layer "F.Cu") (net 24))
 (segment (start 118.7125 149.5) (end 119.2125 150) (width 0.4) (layer "F.Cu") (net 24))
 (segment (start 115.0875 149.5) (end 115.0875 147) (width 0.4) (layer "F.Cu") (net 22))
 (segment (start 187.365 132.115) (end 187.365 133.525) (width 0.4) (layer "F.Cu") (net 1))
 (segment (start 174 126) (end 177 126) (width 0.4) (layer "F.Cu") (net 1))
 (segment (start 177 126) (end 180 129) (width 0.4) (layer "F.Cu") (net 1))
 (segment (start 186.9125 130.1625) (end 186.9125 130.75) (width 0.4) (layer "F.Cu") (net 1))
 (segment (start 186.9125 131.6625) (end 187.365 132.115) (width 0.4) (layer "F.Cu") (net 1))
 (segment (start 185.75 129) (end 186.9125 130.1625) (width 0.4) (layer "F.Cu") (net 1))
 (segment (start 180 129) (end 185.75 129) (width 0.4) (layer "F.Cu") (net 1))
 (segment (start 168.825 124) (end 172 124) (width 0.4) (layer "F.Cu") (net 1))
 (segment (start 186.9125 130.75) (end 186.9125 131.6625) (width 0.4) (layer "F.Cu") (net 1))
 (segment (start 172 124) (end 174 126) (width 0.4) (layer "F.Cu") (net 1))
 (segment (start 127.3375 118.25) (end 125.1625 118.25) (width 1) (layer "F.Cu") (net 20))
 (segment (start 156.4125 149.5) (end 158.5875 149.5) (width 0.2) (layer "F.Cu") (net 11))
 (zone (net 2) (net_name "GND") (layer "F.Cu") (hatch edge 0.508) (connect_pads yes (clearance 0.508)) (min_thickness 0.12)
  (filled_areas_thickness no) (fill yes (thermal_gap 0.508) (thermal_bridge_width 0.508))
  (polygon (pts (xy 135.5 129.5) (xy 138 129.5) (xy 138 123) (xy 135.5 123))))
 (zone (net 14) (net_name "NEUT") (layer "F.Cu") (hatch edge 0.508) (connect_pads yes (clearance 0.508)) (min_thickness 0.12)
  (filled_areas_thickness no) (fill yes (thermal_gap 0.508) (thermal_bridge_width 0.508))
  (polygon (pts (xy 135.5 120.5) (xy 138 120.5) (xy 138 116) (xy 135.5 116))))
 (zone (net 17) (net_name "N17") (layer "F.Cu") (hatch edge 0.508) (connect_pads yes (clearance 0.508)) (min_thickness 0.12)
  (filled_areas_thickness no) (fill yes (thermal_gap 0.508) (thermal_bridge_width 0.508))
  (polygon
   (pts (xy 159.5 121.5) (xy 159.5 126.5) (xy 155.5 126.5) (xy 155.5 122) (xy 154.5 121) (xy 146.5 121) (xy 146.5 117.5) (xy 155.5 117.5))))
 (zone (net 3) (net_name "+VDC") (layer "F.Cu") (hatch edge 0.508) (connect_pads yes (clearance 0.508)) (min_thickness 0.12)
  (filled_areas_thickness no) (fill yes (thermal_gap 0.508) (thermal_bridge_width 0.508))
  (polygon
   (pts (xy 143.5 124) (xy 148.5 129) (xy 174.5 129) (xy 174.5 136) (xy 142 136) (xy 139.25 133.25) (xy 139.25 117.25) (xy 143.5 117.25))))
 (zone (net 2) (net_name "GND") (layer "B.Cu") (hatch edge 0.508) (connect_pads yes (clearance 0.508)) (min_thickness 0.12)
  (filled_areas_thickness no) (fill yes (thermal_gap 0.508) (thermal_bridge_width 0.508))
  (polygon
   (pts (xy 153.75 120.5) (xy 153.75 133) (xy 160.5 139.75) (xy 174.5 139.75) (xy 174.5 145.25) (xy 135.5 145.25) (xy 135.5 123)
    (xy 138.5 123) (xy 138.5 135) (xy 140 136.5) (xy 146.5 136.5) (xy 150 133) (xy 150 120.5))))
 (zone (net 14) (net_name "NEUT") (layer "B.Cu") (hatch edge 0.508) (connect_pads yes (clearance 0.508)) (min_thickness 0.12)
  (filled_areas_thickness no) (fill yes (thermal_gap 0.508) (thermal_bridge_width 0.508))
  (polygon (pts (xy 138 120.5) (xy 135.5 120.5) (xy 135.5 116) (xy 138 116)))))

